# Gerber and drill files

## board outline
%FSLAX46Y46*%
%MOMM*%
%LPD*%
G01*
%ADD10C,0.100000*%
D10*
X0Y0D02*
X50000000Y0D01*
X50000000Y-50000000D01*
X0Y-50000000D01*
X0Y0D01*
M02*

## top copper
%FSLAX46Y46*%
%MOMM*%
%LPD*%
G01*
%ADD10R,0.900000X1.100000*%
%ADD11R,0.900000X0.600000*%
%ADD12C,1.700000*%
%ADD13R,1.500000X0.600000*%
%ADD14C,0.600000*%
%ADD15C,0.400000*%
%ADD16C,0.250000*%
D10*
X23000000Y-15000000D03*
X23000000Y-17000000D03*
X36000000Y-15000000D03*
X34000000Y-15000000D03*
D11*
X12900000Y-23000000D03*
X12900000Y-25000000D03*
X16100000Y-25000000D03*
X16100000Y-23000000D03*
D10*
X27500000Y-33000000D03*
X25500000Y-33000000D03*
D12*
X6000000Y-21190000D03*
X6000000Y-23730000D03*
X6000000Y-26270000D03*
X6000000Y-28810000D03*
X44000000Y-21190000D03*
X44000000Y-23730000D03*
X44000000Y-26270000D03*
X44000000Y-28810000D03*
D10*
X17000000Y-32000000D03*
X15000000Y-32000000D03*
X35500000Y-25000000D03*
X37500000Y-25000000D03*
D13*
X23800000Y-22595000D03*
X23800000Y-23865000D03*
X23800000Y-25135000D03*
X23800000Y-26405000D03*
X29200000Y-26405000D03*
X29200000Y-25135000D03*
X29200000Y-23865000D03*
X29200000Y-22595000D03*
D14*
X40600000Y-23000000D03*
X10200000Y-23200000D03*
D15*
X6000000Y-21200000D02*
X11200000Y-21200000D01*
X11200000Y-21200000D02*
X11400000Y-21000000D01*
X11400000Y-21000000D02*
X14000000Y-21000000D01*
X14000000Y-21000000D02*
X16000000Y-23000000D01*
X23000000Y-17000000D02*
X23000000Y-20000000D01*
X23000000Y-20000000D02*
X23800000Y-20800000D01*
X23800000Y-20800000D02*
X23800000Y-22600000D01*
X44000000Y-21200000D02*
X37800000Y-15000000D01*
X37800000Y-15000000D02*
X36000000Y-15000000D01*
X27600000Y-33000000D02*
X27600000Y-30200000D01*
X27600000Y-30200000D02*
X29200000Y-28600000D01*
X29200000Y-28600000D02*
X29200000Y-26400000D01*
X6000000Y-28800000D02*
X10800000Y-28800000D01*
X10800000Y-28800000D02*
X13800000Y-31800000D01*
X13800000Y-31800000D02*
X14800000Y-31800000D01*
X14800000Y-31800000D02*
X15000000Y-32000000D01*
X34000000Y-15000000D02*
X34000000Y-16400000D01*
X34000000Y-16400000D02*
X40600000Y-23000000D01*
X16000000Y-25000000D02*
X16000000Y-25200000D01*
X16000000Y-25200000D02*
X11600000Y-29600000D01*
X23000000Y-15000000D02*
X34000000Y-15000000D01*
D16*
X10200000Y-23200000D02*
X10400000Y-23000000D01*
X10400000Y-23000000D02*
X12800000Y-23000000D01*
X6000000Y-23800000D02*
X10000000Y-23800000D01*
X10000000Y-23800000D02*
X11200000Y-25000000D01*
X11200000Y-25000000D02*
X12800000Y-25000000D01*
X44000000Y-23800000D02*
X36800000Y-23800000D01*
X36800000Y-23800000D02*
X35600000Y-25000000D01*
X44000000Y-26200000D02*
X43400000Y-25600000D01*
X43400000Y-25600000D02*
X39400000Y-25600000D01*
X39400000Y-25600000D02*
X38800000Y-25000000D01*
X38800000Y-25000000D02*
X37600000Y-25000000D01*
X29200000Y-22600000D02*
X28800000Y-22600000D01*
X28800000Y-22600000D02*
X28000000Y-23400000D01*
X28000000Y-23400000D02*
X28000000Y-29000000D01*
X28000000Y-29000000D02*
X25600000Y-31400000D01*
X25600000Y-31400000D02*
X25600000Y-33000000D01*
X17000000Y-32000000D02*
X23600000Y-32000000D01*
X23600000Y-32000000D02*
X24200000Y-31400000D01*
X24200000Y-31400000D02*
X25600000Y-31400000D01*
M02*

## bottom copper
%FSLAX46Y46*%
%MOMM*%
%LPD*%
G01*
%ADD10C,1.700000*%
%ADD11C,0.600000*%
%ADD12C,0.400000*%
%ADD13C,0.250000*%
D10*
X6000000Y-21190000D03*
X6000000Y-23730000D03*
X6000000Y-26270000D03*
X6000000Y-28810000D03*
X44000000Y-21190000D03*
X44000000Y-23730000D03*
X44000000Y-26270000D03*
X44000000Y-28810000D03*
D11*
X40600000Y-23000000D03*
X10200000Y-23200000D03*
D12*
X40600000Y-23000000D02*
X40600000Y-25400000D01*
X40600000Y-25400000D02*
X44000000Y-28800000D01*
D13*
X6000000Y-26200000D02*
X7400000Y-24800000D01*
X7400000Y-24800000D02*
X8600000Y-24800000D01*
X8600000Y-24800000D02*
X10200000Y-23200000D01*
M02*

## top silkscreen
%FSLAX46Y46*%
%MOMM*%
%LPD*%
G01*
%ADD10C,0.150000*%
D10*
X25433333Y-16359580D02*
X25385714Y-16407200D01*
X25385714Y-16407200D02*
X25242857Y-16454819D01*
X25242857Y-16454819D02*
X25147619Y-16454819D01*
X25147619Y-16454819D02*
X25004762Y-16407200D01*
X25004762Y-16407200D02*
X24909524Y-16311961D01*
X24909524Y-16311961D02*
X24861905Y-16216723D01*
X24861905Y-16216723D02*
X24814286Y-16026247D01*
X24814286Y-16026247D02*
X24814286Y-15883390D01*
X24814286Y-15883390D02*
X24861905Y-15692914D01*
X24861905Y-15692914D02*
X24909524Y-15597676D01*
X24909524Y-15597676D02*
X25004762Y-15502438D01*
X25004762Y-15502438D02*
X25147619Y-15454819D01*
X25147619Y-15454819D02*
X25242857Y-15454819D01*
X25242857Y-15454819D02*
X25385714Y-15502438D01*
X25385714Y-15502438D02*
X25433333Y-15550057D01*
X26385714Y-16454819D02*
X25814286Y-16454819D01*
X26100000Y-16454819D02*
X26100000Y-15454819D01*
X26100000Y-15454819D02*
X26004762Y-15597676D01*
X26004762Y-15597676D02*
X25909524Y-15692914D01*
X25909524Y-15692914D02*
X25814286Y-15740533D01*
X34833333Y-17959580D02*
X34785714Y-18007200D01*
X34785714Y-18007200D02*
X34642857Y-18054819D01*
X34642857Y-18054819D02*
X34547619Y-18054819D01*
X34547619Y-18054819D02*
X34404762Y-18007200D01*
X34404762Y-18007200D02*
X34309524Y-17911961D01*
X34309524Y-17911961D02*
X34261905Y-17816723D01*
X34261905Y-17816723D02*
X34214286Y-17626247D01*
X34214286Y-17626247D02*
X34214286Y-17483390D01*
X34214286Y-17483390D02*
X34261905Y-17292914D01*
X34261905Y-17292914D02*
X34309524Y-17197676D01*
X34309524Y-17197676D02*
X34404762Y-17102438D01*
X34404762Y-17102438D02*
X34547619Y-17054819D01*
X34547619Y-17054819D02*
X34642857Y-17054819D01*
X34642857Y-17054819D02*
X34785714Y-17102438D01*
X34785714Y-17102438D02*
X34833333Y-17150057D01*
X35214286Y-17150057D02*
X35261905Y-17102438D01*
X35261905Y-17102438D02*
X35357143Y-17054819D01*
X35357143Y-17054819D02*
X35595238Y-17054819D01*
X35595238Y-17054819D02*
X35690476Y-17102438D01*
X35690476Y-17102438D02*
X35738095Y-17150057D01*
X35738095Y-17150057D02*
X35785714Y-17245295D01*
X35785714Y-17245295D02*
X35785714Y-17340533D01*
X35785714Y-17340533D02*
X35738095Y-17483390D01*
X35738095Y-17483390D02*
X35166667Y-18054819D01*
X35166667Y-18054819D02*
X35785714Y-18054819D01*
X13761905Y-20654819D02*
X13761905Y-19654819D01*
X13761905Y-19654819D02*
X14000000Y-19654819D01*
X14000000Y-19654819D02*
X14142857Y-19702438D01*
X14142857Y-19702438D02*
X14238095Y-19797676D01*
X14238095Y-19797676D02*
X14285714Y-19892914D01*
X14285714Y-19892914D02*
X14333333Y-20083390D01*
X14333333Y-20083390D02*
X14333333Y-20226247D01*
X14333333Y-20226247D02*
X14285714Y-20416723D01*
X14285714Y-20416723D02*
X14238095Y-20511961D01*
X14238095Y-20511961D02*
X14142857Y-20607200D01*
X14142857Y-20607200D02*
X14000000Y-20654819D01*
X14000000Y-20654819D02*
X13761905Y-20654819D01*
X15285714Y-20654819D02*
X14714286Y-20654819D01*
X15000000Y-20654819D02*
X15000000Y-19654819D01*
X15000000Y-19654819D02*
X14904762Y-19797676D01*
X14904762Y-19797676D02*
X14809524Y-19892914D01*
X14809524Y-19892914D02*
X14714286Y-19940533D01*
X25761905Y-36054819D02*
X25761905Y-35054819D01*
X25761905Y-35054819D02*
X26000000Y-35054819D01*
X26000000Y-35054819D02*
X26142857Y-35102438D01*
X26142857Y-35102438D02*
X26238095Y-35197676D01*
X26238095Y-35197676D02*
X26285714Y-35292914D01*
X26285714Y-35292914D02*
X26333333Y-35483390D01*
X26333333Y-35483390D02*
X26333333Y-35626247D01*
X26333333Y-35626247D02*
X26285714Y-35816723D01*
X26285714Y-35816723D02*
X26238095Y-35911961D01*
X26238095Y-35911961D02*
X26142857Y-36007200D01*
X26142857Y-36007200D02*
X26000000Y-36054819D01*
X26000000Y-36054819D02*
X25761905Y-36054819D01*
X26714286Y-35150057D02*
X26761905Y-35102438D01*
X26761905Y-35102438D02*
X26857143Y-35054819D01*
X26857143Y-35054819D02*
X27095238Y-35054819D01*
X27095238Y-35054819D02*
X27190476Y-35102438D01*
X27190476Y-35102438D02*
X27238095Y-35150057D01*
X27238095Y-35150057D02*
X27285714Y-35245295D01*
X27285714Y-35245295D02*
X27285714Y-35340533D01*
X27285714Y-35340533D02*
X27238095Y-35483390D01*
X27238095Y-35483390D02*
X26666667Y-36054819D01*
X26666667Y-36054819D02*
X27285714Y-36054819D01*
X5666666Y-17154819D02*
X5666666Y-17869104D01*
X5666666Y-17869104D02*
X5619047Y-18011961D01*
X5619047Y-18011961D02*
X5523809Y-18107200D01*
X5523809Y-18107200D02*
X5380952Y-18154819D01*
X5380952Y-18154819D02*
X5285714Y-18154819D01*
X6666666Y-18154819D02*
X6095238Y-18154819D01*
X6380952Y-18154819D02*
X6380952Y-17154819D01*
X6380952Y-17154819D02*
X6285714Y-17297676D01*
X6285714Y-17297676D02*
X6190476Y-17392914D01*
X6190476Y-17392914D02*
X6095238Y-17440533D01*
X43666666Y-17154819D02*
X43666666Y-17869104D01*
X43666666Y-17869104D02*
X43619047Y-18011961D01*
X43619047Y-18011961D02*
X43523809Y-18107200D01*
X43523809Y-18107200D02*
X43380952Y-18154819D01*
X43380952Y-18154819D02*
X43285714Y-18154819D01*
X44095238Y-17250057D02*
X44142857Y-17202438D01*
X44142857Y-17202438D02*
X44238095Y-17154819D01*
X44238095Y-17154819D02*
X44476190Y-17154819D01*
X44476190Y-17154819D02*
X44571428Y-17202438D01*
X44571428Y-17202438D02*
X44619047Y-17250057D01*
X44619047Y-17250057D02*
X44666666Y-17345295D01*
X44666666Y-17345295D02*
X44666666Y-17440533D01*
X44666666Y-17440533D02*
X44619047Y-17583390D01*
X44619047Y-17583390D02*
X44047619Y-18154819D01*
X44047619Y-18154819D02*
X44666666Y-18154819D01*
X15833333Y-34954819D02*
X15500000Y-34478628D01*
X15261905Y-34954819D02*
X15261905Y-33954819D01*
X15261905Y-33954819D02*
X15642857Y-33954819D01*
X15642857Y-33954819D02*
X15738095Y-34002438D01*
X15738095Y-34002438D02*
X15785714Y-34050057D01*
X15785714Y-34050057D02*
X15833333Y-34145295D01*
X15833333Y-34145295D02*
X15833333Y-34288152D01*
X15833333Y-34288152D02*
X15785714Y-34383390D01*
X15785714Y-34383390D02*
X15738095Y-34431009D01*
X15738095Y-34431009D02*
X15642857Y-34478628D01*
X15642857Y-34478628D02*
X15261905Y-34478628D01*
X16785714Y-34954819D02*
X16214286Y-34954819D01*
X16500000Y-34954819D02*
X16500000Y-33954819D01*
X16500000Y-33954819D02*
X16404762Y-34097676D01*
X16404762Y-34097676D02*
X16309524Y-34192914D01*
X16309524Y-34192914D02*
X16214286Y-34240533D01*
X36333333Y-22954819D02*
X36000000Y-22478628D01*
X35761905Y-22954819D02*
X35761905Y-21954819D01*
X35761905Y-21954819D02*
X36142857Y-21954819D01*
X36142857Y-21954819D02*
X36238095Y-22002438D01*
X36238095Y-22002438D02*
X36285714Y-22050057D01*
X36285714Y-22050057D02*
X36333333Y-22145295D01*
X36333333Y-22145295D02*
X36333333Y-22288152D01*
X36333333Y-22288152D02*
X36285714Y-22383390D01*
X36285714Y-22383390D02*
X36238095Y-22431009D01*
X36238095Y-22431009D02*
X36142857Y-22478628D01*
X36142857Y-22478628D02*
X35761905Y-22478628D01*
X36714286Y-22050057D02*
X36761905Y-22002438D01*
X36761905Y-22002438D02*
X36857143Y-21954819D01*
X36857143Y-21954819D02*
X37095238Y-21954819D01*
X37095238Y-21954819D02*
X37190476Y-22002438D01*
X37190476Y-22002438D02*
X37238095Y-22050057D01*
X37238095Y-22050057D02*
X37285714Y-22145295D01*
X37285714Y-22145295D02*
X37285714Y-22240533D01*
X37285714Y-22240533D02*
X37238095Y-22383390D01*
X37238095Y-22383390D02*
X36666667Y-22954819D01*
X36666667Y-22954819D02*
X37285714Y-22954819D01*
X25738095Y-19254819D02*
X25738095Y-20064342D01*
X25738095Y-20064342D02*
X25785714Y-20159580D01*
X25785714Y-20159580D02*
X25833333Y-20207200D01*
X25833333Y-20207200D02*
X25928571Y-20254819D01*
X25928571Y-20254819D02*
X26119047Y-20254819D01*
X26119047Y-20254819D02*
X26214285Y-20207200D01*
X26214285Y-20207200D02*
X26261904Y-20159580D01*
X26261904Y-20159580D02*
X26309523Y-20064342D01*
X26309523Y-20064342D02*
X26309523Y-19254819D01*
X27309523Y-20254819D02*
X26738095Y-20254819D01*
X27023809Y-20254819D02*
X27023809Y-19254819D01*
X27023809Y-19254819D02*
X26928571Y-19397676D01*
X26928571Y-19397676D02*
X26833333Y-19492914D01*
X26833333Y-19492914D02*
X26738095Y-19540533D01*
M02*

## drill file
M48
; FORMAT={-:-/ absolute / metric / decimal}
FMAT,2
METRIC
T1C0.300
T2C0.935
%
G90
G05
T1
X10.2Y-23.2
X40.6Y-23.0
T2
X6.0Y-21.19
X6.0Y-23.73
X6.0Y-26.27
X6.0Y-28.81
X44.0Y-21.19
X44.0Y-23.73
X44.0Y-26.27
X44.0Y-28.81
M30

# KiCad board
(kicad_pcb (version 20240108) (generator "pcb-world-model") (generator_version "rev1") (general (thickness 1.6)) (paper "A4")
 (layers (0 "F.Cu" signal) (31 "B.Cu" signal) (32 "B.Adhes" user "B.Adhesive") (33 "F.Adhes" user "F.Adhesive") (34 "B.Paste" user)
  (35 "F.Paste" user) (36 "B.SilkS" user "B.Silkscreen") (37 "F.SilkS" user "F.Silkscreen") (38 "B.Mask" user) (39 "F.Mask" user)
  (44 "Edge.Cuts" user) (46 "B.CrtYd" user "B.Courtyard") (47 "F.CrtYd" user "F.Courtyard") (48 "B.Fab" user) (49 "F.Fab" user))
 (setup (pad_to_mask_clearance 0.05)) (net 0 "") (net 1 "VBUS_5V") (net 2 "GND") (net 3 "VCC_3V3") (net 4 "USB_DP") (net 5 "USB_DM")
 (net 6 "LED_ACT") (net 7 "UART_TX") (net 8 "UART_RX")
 (gr_rect (start 0.0 0.0) (end 50.0000 50.0000) (stroke (width 0.1) (type default)) (fill none) (layer "Edge.Cuts"))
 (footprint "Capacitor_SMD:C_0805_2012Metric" (layer "F.Cu") (at 23.0000 16.0000 270)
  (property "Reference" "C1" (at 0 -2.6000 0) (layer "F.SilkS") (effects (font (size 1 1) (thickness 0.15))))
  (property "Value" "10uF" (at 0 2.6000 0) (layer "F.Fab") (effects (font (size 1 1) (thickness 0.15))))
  (pad "1" smd rect (at -1.0000 0.0000) (size 0.9000 1.1000) (layers "F.Cu" "F.Paste" "F.Mask") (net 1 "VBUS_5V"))
  (pad "2" smd rect (at 1.0000 0.0000) (size 0.9000 1.1000) (layers "F.Cu" "F.Paste" "F.Mask") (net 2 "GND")))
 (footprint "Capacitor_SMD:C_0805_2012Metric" (layer "F.Cu") (at 35.0000 15.0000 180)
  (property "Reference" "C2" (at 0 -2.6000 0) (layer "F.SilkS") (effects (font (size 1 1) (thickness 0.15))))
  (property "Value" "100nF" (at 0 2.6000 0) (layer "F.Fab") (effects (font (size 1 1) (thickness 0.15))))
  (pad "1" smd rect (at -1.0000 0.0000) (size 0.9000 1.1000) (layers "F.Cu" "F.Paste" "F.Mask") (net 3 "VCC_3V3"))
  (pad "2" smd rect (at 1.0000 0.0000) (size 0.9000 1.1000) (layers "F.Cu" "F.Paste" "F.Mask") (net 2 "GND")))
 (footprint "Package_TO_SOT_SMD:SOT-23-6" (layer "F.Cu") (at 14.5000 24.0000 0)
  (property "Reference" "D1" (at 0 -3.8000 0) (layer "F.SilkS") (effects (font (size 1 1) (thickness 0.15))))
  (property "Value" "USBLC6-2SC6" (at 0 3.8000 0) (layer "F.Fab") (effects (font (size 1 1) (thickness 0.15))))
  (pad "1" smd rect (at -1.6000 -1.0000) (size 0.9000 0.6000) (layers "F.Cu" "F.Paste" "F.Mask") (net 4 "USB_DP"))
  (pad "2" smd rect (at -1.6000 1.0000) (size 0.9000 0.6000) (layers "F.Cu" "F.Paste" "F.Mask") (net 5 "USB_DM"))
  (pad "3" smd rect (at 1.6000 1.0000) (size 0.9000 0.6000) (layers "F.Cu" "F.Paste" "F.Mask") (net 2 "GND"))
  (pad "4" smd rect (at 1.6000 -1.0000) (size 0.9000 0.6000) (layers "F.Cu" "F.Paste" "F.Mask") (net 1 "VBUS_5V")))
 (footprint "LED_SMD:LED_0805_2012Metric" (layer "F.Cu") (at 26.5000 33.0000 180)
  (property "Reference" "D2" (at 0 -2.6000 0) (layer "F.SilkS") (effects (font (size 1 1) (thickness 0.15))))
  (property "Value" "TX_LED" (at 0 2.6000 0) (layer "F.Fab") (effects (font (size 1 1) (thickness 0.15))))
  (pad "1" smd rect (at -1.0000 0.0000) (size 0.9000 1.1000) (layers "F.Cu" "F.Paste" "F.Mask") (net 3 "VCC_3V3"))
  (pad "2" smd rect (at 1.0000 0.0000) (size 0.9000 1.1000) (layers "F.Cu" "F.Paste" "F.Mask") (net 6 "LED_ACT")))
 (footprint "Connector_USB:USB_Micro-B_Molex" (layer "F.Cu") (at 6.0000 25.0000 0) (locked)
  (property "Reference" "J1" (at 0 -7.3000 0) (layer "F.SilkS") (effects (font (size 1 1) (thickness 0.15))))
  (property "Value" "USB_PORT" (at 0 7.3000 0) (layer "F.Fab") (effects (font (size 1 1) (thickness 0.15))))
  (pad "1" thru_hole circle (at 0.0000 -3.8100) (size 1.7000 1.7000) (drill 0.9350) (layers "*.Cu" "*.Mask") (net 1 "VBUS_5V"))
  (pad "2" thru_hole circle (at 0.0000 -1.2700) (size 1.7000 1.7000) (drill 0.9350) (layers "*.Cu" "*.Mask") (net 5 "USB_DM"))
  (pad "3" thru_hole circle (at 0.0000 1.2700) (size 1.7000 1.7000) (drill 0.9350) (layers "*.Cu" "*.Mask") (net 4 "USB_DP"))
  (pad "4" thru_hole circle (at 0.0000 3.8100) (size 1.7000 1.7000) (drill 0.9350) (layers "*.Cu" "*.Mask") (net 2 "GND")))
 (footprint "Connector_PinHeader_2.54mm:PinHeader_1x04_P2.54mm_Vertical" (layer "F.Cu") (at 44.0000 25.0000 0) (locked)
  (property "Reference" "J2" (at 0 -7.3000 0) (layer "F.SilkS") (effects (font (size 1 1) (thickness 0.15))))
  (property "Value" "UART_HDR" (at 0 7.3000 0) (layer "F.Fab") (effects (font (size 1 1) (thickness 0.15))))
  (pad "1" thru_hole circle (at 0.0000 -3.8100) (size 1.7000 1.7000) (drill 0.9350) (layers "*.Cu" "*.Mask") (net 3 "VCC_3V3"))
  (pad "2" thru_hole circle (at 0.0000 -1.2700) (size 1.7000 1.7000) (drill 0.9350) (layers "*.Cu" "*.Mask") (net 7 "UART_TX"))
  (pad "3" thru_hole circle (at 0.0000 1.2700) (size 1.7000 1.7000) (drill 0.9350) (layers "*.Cu" "*.Mask") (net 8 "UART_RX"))
  (pad "4" thru_hole circle (at 0.0000 3.8100) (size 1.7000 1.7000) (drill 0.9350) (layers "*.Cu" "*.Mask") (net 2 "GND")))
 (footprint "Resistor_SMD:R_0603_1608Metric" (layer "F.Cu") (at 16.0000 32.0000 180)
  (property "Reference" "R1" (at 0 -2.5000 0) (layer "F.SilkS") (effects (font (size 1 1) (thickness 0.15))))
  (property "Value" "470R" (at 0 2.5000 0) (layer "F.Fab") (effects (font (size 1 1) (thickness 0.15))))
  (pad "1" smd rect (at -1.0000 0.0000) (size 0.9000 1.1000) (layers "F.Cu" "F.Paste" "F.Mask") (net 6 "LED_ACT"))
  (pad "2" smd rect (at 1.0000 0.0000) (size 0.9000 1.1000) (layers "F.Cu" "F.Paste" "F.Mask") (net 2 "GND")))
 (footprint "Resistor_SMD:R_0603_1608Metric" (layer "F.Cu") (at 36.5000 25.0000 0)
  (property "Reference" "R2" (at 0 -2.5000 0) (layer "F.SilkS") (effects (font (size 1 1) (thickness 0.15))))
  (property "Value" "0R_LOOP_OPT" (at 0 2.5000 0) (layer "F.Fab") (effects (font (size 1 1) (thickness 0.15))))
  (pad "1" smd rect (at -1.0000 0.0000) (size 0.9000 1.1000) (layers "F.Cu" "F.Paste" "F.Mask") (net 7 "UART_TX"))
  (pad "2" smd rect (at 1.0000 0.0000) (size 0.9000 1.1000) (layers "F.Cu" "F.Paste" "F.Mask") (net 8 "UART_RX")))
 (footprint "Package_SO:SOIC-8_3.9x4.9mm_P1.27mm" (layer "F.Cu") (at 26.5000 24.5000 0)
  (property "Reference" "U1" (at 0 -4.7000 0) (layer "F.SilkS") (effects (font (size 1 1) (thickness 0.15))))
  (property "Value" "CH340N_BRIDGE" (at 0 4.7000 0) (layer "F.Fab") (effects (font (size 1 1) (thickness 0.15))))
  (pad "1" smd rect (at -2.7000 -1.9050) (size 1.5000 0.6000) (layers "F.Cu" "F.Paste" "F.Mask") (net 1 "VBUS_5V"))
  (pad "2" smd rect (at -2.7000 -0.6350) (size 1.5000 0.6000) (layers "F.Cu" "F.Paste" "F.Mask") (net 4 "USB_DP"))
  (pad "3" smd rect (at -2.7000 0.6350) (size 1.5000 0.6000) (layers "F.Cu" "F.Paste" "F.Mask") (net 5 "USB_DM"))
  (pad "4" smd rect (at -2.7000 1.9050) (size 1.5000 0.6000) (layers "F.Cu" "F.Paste" "F.Mask") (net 2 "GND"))
  (pad "5" smd rect (at 2.7000 1.9050) (size 1.5000 0.6000) (layers "F.Cu" "F.Paste" "F.Mask") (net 3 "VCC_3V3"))
  (pad "6" smd rect (at 2.7000 0.6350) (size 1.5000 0.6000) (layers "F.Cu" "F.Paste" "F.Mask") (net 7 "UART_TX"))
  (pad "7" smd rect (at 2.7000 -0.6350) (size 1.5000 0.6000) (layers "F.Cu" "F.Paste" "F.Mask") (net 8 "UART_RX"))
  (pad "8" smd rect (at 2.7000 -1.9050) (size 1.5000 0.6000) (layers "F.Cu" "F.Paste" "F.Mask") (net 6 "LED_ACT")))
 (segment (start 6.0000 21.2000) (end 11.2000 21.2000) (width 0.4000) (layer "F.Cu") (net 1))
 (segment (start 11.2000 21.2000) (end 11.4000 21.0000) (width 0.4000) (layer "F.Cu") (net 1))
 (segment (start 11.4000 21.0000) (end 14.0000 21.0000) (width 0.4000) (layer "F.Cu") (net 1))
 (segment (start 14.0000 21.0000) (end 16.0000 23.0000) (width 0.4000) (layer "F.Cu") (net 1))
 (segment (start 23.0000 17.0000) (end 23.0000 20.0000) (width 0.4000) (layer "F.Cu") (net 1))
 (segment (start 23.0000 20.0000) (end 23.8000 20.8000) (width 0.4000) (layer "F.Cu") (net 1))
 (segment (start 23.8000 20.8000) (end 23.8000 22.6000) (width 0.4000) (layer "F.Cu") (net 1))
 (segment (start 44.0000 21.2000) (end 37.8000 15.0000) (width 0.4000) (layer "F.Cu") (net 3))
 (segment (start 37.8000 15.0000) (end 36.0000 15.0000) (width 0.4000) (layer "F.Cu") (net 3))
 (segment (start 27.6000 33.0000) (end 27.6000 30.2000) (width 0.4000) (layer "F.Cu") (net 3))
 (segment (start 27.6000 30.2000) (end 29.2000 28.6000) (width 0.4000) (layer "F.Cu") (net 3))
 (segment (start 29.2000 28.6000) (end 29.2000 26.4000) (width 0.4000) (layer "F.Cu") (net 3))
 (segment (start 6.0000 28.8000) (end 10.8000 28.8000) (width 0.4000) (layer "F.Cu") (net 2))
 (segment (start 10.8000 28.8000) (end 13.8000 31.8000) (width 0.4000) (layer "F.Cu") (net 2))
 (segment (start 13.8000 31.8000) (end 14.8000 31.8000) (width 0.4000) (layer "F.Cu") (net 2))
 (segment (start 14.8000 31.8000) (end 15.0000 32.0000) (width 0.4000) (layer "F.Cu") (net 2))
 (segment (start 34.0000 15.0000) (end 34.0000 16.4000) (width 0.4000) (layer "F.Cu") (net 2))
 (segment (start 34.0000 16.4000) (end 40.6000 23.0000) (width 0.4000) (layer "F.Cu") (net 2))
 (segment (start 40.6000 23.0000) (end 40.6000 25.4000) (width 0.4000) (layer "B.Cu") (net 2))
 (segment (start 40.6000 25.4000) (end 44.0000 28.8000) (width 0.4000) (layer "B.Cu") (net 2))
 (segment (start 16.0000 25.0000) (end 16.0000 25.2000) (width 0.4000) (layer "F.Cu") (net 2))
 (segment (start 16.0000 25.2000) (end 11.6000 29.6000) (width 0.4000) (layer "F.Cu") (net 2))
 (segment (start 23.0000 15.0000) (end 34.0000 15.0000) (width 0.4000) (layer "F.Cu") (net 2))
 (segment (start 6.0000 26.2000) (end 7.4000 24.8000) (width 0.2500) (layer "B.Cu") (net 4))
 (segment (start 7.4000 24.8000) (end 8.6000 24.8000) (width 0.2500) (layer "B.Cu") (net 4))
 (segment (start 8.6000 24.8000) (end 10.2000 23.2000) (width 0.2500) (layer "B.Cu") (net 4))
 (segment (start 10.2000 23.2000) (end 10.4000 23.0000) (width 0.2500) (layer "F.Cu") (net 4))
 (segment (start 10.4000 23.0000) (end 12.8000 23.0000) (width 0.2500) (layer "F.Cu") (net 4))
 (segment (start 6.0000 23.8000) (end 10.0000 23.8000) (width 0.2500) (layer "F.Cu") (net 5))
 (segment (start 10.0000 23.8000) (end 11.2000 25.0000) (width 0.2500) (layer "F.Cu") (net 5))
 (segment (start 11.2000 25.0000) (end 12.8000 25.0000) (width 0.2500) (layer "F.Cu") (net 5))
 (segment (start 44.0000 23.8000) (end 36.8000 23.8000) (width 0.2500) (layer "F.Cu") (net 7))
 (segment (start 36.8000 23.8000) (end 35.6000 25.0000) (width 0.2500) (layer "F.Cu") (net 7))
 (segment (start 44.0000 26.2000) (end 43.4000 25.6000) (width 0.2500) (layer "F.Cu") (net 8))
 (segment (start 43.4000 25.6000) (end 39.4000 25.6000) (width 0.2500) (layer "F.Cu") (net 8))
 (segment (start 39.4000 25.6000) (end 38.8000 25.0000) (width 0.2500) (layer "F.Cu") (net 8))
 (segment (start 38.8000 25.0000) (end 37.6000 25.0000) (width 0.2500) (layer "F.Cu") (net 8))
 (segment (start 29.2000 22.6000) (end 28.8000 22.6000) (width 0.2500) (layer "F.Cu") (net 6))
 (segment (start 28.8000 22.6000) (end 28.0000 23.4000) (width 0.2500) (layer "F.Cu") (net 6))
 (segment (start 28.0000 23.4000) (end 28.0000 29.0000) (width 0.2500) (layer "F.Cu") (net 6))
 (segment (start 28.0000 29.0000) (end 25.6000 31.4000) (width 0.2500) (layer "F.Cu") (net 6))
 (segment (start 25.6000 31.4000) (end 25.6000 33.0000) (width 0.2500) (layer "F.Cu") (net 6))
 (segment (start 17.0000 32.0000) (end 23.6000 32.0000) (width 0.2500) (layer "F.Cu") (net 6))
 (segment (start 23.6000 32.0000) (end 24.2000 31.4000) (width 0.2500) (layer "F.Cu") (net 6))
 (segment (start 24.2000 31.4000) (end 25.6000 31.4000) (width 0.2500) (layer "F.Cu") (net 6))
 (via (at 40.6000 23.0000) (size 0.6000) (drill 0.3000) (layers "F.Cu" "B.Cu") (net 2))
 (via (at 10.2000 23.2000) (size 0.6000) (drill 0.3000) (layers "F.Cu" "B.Cu") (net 4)))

